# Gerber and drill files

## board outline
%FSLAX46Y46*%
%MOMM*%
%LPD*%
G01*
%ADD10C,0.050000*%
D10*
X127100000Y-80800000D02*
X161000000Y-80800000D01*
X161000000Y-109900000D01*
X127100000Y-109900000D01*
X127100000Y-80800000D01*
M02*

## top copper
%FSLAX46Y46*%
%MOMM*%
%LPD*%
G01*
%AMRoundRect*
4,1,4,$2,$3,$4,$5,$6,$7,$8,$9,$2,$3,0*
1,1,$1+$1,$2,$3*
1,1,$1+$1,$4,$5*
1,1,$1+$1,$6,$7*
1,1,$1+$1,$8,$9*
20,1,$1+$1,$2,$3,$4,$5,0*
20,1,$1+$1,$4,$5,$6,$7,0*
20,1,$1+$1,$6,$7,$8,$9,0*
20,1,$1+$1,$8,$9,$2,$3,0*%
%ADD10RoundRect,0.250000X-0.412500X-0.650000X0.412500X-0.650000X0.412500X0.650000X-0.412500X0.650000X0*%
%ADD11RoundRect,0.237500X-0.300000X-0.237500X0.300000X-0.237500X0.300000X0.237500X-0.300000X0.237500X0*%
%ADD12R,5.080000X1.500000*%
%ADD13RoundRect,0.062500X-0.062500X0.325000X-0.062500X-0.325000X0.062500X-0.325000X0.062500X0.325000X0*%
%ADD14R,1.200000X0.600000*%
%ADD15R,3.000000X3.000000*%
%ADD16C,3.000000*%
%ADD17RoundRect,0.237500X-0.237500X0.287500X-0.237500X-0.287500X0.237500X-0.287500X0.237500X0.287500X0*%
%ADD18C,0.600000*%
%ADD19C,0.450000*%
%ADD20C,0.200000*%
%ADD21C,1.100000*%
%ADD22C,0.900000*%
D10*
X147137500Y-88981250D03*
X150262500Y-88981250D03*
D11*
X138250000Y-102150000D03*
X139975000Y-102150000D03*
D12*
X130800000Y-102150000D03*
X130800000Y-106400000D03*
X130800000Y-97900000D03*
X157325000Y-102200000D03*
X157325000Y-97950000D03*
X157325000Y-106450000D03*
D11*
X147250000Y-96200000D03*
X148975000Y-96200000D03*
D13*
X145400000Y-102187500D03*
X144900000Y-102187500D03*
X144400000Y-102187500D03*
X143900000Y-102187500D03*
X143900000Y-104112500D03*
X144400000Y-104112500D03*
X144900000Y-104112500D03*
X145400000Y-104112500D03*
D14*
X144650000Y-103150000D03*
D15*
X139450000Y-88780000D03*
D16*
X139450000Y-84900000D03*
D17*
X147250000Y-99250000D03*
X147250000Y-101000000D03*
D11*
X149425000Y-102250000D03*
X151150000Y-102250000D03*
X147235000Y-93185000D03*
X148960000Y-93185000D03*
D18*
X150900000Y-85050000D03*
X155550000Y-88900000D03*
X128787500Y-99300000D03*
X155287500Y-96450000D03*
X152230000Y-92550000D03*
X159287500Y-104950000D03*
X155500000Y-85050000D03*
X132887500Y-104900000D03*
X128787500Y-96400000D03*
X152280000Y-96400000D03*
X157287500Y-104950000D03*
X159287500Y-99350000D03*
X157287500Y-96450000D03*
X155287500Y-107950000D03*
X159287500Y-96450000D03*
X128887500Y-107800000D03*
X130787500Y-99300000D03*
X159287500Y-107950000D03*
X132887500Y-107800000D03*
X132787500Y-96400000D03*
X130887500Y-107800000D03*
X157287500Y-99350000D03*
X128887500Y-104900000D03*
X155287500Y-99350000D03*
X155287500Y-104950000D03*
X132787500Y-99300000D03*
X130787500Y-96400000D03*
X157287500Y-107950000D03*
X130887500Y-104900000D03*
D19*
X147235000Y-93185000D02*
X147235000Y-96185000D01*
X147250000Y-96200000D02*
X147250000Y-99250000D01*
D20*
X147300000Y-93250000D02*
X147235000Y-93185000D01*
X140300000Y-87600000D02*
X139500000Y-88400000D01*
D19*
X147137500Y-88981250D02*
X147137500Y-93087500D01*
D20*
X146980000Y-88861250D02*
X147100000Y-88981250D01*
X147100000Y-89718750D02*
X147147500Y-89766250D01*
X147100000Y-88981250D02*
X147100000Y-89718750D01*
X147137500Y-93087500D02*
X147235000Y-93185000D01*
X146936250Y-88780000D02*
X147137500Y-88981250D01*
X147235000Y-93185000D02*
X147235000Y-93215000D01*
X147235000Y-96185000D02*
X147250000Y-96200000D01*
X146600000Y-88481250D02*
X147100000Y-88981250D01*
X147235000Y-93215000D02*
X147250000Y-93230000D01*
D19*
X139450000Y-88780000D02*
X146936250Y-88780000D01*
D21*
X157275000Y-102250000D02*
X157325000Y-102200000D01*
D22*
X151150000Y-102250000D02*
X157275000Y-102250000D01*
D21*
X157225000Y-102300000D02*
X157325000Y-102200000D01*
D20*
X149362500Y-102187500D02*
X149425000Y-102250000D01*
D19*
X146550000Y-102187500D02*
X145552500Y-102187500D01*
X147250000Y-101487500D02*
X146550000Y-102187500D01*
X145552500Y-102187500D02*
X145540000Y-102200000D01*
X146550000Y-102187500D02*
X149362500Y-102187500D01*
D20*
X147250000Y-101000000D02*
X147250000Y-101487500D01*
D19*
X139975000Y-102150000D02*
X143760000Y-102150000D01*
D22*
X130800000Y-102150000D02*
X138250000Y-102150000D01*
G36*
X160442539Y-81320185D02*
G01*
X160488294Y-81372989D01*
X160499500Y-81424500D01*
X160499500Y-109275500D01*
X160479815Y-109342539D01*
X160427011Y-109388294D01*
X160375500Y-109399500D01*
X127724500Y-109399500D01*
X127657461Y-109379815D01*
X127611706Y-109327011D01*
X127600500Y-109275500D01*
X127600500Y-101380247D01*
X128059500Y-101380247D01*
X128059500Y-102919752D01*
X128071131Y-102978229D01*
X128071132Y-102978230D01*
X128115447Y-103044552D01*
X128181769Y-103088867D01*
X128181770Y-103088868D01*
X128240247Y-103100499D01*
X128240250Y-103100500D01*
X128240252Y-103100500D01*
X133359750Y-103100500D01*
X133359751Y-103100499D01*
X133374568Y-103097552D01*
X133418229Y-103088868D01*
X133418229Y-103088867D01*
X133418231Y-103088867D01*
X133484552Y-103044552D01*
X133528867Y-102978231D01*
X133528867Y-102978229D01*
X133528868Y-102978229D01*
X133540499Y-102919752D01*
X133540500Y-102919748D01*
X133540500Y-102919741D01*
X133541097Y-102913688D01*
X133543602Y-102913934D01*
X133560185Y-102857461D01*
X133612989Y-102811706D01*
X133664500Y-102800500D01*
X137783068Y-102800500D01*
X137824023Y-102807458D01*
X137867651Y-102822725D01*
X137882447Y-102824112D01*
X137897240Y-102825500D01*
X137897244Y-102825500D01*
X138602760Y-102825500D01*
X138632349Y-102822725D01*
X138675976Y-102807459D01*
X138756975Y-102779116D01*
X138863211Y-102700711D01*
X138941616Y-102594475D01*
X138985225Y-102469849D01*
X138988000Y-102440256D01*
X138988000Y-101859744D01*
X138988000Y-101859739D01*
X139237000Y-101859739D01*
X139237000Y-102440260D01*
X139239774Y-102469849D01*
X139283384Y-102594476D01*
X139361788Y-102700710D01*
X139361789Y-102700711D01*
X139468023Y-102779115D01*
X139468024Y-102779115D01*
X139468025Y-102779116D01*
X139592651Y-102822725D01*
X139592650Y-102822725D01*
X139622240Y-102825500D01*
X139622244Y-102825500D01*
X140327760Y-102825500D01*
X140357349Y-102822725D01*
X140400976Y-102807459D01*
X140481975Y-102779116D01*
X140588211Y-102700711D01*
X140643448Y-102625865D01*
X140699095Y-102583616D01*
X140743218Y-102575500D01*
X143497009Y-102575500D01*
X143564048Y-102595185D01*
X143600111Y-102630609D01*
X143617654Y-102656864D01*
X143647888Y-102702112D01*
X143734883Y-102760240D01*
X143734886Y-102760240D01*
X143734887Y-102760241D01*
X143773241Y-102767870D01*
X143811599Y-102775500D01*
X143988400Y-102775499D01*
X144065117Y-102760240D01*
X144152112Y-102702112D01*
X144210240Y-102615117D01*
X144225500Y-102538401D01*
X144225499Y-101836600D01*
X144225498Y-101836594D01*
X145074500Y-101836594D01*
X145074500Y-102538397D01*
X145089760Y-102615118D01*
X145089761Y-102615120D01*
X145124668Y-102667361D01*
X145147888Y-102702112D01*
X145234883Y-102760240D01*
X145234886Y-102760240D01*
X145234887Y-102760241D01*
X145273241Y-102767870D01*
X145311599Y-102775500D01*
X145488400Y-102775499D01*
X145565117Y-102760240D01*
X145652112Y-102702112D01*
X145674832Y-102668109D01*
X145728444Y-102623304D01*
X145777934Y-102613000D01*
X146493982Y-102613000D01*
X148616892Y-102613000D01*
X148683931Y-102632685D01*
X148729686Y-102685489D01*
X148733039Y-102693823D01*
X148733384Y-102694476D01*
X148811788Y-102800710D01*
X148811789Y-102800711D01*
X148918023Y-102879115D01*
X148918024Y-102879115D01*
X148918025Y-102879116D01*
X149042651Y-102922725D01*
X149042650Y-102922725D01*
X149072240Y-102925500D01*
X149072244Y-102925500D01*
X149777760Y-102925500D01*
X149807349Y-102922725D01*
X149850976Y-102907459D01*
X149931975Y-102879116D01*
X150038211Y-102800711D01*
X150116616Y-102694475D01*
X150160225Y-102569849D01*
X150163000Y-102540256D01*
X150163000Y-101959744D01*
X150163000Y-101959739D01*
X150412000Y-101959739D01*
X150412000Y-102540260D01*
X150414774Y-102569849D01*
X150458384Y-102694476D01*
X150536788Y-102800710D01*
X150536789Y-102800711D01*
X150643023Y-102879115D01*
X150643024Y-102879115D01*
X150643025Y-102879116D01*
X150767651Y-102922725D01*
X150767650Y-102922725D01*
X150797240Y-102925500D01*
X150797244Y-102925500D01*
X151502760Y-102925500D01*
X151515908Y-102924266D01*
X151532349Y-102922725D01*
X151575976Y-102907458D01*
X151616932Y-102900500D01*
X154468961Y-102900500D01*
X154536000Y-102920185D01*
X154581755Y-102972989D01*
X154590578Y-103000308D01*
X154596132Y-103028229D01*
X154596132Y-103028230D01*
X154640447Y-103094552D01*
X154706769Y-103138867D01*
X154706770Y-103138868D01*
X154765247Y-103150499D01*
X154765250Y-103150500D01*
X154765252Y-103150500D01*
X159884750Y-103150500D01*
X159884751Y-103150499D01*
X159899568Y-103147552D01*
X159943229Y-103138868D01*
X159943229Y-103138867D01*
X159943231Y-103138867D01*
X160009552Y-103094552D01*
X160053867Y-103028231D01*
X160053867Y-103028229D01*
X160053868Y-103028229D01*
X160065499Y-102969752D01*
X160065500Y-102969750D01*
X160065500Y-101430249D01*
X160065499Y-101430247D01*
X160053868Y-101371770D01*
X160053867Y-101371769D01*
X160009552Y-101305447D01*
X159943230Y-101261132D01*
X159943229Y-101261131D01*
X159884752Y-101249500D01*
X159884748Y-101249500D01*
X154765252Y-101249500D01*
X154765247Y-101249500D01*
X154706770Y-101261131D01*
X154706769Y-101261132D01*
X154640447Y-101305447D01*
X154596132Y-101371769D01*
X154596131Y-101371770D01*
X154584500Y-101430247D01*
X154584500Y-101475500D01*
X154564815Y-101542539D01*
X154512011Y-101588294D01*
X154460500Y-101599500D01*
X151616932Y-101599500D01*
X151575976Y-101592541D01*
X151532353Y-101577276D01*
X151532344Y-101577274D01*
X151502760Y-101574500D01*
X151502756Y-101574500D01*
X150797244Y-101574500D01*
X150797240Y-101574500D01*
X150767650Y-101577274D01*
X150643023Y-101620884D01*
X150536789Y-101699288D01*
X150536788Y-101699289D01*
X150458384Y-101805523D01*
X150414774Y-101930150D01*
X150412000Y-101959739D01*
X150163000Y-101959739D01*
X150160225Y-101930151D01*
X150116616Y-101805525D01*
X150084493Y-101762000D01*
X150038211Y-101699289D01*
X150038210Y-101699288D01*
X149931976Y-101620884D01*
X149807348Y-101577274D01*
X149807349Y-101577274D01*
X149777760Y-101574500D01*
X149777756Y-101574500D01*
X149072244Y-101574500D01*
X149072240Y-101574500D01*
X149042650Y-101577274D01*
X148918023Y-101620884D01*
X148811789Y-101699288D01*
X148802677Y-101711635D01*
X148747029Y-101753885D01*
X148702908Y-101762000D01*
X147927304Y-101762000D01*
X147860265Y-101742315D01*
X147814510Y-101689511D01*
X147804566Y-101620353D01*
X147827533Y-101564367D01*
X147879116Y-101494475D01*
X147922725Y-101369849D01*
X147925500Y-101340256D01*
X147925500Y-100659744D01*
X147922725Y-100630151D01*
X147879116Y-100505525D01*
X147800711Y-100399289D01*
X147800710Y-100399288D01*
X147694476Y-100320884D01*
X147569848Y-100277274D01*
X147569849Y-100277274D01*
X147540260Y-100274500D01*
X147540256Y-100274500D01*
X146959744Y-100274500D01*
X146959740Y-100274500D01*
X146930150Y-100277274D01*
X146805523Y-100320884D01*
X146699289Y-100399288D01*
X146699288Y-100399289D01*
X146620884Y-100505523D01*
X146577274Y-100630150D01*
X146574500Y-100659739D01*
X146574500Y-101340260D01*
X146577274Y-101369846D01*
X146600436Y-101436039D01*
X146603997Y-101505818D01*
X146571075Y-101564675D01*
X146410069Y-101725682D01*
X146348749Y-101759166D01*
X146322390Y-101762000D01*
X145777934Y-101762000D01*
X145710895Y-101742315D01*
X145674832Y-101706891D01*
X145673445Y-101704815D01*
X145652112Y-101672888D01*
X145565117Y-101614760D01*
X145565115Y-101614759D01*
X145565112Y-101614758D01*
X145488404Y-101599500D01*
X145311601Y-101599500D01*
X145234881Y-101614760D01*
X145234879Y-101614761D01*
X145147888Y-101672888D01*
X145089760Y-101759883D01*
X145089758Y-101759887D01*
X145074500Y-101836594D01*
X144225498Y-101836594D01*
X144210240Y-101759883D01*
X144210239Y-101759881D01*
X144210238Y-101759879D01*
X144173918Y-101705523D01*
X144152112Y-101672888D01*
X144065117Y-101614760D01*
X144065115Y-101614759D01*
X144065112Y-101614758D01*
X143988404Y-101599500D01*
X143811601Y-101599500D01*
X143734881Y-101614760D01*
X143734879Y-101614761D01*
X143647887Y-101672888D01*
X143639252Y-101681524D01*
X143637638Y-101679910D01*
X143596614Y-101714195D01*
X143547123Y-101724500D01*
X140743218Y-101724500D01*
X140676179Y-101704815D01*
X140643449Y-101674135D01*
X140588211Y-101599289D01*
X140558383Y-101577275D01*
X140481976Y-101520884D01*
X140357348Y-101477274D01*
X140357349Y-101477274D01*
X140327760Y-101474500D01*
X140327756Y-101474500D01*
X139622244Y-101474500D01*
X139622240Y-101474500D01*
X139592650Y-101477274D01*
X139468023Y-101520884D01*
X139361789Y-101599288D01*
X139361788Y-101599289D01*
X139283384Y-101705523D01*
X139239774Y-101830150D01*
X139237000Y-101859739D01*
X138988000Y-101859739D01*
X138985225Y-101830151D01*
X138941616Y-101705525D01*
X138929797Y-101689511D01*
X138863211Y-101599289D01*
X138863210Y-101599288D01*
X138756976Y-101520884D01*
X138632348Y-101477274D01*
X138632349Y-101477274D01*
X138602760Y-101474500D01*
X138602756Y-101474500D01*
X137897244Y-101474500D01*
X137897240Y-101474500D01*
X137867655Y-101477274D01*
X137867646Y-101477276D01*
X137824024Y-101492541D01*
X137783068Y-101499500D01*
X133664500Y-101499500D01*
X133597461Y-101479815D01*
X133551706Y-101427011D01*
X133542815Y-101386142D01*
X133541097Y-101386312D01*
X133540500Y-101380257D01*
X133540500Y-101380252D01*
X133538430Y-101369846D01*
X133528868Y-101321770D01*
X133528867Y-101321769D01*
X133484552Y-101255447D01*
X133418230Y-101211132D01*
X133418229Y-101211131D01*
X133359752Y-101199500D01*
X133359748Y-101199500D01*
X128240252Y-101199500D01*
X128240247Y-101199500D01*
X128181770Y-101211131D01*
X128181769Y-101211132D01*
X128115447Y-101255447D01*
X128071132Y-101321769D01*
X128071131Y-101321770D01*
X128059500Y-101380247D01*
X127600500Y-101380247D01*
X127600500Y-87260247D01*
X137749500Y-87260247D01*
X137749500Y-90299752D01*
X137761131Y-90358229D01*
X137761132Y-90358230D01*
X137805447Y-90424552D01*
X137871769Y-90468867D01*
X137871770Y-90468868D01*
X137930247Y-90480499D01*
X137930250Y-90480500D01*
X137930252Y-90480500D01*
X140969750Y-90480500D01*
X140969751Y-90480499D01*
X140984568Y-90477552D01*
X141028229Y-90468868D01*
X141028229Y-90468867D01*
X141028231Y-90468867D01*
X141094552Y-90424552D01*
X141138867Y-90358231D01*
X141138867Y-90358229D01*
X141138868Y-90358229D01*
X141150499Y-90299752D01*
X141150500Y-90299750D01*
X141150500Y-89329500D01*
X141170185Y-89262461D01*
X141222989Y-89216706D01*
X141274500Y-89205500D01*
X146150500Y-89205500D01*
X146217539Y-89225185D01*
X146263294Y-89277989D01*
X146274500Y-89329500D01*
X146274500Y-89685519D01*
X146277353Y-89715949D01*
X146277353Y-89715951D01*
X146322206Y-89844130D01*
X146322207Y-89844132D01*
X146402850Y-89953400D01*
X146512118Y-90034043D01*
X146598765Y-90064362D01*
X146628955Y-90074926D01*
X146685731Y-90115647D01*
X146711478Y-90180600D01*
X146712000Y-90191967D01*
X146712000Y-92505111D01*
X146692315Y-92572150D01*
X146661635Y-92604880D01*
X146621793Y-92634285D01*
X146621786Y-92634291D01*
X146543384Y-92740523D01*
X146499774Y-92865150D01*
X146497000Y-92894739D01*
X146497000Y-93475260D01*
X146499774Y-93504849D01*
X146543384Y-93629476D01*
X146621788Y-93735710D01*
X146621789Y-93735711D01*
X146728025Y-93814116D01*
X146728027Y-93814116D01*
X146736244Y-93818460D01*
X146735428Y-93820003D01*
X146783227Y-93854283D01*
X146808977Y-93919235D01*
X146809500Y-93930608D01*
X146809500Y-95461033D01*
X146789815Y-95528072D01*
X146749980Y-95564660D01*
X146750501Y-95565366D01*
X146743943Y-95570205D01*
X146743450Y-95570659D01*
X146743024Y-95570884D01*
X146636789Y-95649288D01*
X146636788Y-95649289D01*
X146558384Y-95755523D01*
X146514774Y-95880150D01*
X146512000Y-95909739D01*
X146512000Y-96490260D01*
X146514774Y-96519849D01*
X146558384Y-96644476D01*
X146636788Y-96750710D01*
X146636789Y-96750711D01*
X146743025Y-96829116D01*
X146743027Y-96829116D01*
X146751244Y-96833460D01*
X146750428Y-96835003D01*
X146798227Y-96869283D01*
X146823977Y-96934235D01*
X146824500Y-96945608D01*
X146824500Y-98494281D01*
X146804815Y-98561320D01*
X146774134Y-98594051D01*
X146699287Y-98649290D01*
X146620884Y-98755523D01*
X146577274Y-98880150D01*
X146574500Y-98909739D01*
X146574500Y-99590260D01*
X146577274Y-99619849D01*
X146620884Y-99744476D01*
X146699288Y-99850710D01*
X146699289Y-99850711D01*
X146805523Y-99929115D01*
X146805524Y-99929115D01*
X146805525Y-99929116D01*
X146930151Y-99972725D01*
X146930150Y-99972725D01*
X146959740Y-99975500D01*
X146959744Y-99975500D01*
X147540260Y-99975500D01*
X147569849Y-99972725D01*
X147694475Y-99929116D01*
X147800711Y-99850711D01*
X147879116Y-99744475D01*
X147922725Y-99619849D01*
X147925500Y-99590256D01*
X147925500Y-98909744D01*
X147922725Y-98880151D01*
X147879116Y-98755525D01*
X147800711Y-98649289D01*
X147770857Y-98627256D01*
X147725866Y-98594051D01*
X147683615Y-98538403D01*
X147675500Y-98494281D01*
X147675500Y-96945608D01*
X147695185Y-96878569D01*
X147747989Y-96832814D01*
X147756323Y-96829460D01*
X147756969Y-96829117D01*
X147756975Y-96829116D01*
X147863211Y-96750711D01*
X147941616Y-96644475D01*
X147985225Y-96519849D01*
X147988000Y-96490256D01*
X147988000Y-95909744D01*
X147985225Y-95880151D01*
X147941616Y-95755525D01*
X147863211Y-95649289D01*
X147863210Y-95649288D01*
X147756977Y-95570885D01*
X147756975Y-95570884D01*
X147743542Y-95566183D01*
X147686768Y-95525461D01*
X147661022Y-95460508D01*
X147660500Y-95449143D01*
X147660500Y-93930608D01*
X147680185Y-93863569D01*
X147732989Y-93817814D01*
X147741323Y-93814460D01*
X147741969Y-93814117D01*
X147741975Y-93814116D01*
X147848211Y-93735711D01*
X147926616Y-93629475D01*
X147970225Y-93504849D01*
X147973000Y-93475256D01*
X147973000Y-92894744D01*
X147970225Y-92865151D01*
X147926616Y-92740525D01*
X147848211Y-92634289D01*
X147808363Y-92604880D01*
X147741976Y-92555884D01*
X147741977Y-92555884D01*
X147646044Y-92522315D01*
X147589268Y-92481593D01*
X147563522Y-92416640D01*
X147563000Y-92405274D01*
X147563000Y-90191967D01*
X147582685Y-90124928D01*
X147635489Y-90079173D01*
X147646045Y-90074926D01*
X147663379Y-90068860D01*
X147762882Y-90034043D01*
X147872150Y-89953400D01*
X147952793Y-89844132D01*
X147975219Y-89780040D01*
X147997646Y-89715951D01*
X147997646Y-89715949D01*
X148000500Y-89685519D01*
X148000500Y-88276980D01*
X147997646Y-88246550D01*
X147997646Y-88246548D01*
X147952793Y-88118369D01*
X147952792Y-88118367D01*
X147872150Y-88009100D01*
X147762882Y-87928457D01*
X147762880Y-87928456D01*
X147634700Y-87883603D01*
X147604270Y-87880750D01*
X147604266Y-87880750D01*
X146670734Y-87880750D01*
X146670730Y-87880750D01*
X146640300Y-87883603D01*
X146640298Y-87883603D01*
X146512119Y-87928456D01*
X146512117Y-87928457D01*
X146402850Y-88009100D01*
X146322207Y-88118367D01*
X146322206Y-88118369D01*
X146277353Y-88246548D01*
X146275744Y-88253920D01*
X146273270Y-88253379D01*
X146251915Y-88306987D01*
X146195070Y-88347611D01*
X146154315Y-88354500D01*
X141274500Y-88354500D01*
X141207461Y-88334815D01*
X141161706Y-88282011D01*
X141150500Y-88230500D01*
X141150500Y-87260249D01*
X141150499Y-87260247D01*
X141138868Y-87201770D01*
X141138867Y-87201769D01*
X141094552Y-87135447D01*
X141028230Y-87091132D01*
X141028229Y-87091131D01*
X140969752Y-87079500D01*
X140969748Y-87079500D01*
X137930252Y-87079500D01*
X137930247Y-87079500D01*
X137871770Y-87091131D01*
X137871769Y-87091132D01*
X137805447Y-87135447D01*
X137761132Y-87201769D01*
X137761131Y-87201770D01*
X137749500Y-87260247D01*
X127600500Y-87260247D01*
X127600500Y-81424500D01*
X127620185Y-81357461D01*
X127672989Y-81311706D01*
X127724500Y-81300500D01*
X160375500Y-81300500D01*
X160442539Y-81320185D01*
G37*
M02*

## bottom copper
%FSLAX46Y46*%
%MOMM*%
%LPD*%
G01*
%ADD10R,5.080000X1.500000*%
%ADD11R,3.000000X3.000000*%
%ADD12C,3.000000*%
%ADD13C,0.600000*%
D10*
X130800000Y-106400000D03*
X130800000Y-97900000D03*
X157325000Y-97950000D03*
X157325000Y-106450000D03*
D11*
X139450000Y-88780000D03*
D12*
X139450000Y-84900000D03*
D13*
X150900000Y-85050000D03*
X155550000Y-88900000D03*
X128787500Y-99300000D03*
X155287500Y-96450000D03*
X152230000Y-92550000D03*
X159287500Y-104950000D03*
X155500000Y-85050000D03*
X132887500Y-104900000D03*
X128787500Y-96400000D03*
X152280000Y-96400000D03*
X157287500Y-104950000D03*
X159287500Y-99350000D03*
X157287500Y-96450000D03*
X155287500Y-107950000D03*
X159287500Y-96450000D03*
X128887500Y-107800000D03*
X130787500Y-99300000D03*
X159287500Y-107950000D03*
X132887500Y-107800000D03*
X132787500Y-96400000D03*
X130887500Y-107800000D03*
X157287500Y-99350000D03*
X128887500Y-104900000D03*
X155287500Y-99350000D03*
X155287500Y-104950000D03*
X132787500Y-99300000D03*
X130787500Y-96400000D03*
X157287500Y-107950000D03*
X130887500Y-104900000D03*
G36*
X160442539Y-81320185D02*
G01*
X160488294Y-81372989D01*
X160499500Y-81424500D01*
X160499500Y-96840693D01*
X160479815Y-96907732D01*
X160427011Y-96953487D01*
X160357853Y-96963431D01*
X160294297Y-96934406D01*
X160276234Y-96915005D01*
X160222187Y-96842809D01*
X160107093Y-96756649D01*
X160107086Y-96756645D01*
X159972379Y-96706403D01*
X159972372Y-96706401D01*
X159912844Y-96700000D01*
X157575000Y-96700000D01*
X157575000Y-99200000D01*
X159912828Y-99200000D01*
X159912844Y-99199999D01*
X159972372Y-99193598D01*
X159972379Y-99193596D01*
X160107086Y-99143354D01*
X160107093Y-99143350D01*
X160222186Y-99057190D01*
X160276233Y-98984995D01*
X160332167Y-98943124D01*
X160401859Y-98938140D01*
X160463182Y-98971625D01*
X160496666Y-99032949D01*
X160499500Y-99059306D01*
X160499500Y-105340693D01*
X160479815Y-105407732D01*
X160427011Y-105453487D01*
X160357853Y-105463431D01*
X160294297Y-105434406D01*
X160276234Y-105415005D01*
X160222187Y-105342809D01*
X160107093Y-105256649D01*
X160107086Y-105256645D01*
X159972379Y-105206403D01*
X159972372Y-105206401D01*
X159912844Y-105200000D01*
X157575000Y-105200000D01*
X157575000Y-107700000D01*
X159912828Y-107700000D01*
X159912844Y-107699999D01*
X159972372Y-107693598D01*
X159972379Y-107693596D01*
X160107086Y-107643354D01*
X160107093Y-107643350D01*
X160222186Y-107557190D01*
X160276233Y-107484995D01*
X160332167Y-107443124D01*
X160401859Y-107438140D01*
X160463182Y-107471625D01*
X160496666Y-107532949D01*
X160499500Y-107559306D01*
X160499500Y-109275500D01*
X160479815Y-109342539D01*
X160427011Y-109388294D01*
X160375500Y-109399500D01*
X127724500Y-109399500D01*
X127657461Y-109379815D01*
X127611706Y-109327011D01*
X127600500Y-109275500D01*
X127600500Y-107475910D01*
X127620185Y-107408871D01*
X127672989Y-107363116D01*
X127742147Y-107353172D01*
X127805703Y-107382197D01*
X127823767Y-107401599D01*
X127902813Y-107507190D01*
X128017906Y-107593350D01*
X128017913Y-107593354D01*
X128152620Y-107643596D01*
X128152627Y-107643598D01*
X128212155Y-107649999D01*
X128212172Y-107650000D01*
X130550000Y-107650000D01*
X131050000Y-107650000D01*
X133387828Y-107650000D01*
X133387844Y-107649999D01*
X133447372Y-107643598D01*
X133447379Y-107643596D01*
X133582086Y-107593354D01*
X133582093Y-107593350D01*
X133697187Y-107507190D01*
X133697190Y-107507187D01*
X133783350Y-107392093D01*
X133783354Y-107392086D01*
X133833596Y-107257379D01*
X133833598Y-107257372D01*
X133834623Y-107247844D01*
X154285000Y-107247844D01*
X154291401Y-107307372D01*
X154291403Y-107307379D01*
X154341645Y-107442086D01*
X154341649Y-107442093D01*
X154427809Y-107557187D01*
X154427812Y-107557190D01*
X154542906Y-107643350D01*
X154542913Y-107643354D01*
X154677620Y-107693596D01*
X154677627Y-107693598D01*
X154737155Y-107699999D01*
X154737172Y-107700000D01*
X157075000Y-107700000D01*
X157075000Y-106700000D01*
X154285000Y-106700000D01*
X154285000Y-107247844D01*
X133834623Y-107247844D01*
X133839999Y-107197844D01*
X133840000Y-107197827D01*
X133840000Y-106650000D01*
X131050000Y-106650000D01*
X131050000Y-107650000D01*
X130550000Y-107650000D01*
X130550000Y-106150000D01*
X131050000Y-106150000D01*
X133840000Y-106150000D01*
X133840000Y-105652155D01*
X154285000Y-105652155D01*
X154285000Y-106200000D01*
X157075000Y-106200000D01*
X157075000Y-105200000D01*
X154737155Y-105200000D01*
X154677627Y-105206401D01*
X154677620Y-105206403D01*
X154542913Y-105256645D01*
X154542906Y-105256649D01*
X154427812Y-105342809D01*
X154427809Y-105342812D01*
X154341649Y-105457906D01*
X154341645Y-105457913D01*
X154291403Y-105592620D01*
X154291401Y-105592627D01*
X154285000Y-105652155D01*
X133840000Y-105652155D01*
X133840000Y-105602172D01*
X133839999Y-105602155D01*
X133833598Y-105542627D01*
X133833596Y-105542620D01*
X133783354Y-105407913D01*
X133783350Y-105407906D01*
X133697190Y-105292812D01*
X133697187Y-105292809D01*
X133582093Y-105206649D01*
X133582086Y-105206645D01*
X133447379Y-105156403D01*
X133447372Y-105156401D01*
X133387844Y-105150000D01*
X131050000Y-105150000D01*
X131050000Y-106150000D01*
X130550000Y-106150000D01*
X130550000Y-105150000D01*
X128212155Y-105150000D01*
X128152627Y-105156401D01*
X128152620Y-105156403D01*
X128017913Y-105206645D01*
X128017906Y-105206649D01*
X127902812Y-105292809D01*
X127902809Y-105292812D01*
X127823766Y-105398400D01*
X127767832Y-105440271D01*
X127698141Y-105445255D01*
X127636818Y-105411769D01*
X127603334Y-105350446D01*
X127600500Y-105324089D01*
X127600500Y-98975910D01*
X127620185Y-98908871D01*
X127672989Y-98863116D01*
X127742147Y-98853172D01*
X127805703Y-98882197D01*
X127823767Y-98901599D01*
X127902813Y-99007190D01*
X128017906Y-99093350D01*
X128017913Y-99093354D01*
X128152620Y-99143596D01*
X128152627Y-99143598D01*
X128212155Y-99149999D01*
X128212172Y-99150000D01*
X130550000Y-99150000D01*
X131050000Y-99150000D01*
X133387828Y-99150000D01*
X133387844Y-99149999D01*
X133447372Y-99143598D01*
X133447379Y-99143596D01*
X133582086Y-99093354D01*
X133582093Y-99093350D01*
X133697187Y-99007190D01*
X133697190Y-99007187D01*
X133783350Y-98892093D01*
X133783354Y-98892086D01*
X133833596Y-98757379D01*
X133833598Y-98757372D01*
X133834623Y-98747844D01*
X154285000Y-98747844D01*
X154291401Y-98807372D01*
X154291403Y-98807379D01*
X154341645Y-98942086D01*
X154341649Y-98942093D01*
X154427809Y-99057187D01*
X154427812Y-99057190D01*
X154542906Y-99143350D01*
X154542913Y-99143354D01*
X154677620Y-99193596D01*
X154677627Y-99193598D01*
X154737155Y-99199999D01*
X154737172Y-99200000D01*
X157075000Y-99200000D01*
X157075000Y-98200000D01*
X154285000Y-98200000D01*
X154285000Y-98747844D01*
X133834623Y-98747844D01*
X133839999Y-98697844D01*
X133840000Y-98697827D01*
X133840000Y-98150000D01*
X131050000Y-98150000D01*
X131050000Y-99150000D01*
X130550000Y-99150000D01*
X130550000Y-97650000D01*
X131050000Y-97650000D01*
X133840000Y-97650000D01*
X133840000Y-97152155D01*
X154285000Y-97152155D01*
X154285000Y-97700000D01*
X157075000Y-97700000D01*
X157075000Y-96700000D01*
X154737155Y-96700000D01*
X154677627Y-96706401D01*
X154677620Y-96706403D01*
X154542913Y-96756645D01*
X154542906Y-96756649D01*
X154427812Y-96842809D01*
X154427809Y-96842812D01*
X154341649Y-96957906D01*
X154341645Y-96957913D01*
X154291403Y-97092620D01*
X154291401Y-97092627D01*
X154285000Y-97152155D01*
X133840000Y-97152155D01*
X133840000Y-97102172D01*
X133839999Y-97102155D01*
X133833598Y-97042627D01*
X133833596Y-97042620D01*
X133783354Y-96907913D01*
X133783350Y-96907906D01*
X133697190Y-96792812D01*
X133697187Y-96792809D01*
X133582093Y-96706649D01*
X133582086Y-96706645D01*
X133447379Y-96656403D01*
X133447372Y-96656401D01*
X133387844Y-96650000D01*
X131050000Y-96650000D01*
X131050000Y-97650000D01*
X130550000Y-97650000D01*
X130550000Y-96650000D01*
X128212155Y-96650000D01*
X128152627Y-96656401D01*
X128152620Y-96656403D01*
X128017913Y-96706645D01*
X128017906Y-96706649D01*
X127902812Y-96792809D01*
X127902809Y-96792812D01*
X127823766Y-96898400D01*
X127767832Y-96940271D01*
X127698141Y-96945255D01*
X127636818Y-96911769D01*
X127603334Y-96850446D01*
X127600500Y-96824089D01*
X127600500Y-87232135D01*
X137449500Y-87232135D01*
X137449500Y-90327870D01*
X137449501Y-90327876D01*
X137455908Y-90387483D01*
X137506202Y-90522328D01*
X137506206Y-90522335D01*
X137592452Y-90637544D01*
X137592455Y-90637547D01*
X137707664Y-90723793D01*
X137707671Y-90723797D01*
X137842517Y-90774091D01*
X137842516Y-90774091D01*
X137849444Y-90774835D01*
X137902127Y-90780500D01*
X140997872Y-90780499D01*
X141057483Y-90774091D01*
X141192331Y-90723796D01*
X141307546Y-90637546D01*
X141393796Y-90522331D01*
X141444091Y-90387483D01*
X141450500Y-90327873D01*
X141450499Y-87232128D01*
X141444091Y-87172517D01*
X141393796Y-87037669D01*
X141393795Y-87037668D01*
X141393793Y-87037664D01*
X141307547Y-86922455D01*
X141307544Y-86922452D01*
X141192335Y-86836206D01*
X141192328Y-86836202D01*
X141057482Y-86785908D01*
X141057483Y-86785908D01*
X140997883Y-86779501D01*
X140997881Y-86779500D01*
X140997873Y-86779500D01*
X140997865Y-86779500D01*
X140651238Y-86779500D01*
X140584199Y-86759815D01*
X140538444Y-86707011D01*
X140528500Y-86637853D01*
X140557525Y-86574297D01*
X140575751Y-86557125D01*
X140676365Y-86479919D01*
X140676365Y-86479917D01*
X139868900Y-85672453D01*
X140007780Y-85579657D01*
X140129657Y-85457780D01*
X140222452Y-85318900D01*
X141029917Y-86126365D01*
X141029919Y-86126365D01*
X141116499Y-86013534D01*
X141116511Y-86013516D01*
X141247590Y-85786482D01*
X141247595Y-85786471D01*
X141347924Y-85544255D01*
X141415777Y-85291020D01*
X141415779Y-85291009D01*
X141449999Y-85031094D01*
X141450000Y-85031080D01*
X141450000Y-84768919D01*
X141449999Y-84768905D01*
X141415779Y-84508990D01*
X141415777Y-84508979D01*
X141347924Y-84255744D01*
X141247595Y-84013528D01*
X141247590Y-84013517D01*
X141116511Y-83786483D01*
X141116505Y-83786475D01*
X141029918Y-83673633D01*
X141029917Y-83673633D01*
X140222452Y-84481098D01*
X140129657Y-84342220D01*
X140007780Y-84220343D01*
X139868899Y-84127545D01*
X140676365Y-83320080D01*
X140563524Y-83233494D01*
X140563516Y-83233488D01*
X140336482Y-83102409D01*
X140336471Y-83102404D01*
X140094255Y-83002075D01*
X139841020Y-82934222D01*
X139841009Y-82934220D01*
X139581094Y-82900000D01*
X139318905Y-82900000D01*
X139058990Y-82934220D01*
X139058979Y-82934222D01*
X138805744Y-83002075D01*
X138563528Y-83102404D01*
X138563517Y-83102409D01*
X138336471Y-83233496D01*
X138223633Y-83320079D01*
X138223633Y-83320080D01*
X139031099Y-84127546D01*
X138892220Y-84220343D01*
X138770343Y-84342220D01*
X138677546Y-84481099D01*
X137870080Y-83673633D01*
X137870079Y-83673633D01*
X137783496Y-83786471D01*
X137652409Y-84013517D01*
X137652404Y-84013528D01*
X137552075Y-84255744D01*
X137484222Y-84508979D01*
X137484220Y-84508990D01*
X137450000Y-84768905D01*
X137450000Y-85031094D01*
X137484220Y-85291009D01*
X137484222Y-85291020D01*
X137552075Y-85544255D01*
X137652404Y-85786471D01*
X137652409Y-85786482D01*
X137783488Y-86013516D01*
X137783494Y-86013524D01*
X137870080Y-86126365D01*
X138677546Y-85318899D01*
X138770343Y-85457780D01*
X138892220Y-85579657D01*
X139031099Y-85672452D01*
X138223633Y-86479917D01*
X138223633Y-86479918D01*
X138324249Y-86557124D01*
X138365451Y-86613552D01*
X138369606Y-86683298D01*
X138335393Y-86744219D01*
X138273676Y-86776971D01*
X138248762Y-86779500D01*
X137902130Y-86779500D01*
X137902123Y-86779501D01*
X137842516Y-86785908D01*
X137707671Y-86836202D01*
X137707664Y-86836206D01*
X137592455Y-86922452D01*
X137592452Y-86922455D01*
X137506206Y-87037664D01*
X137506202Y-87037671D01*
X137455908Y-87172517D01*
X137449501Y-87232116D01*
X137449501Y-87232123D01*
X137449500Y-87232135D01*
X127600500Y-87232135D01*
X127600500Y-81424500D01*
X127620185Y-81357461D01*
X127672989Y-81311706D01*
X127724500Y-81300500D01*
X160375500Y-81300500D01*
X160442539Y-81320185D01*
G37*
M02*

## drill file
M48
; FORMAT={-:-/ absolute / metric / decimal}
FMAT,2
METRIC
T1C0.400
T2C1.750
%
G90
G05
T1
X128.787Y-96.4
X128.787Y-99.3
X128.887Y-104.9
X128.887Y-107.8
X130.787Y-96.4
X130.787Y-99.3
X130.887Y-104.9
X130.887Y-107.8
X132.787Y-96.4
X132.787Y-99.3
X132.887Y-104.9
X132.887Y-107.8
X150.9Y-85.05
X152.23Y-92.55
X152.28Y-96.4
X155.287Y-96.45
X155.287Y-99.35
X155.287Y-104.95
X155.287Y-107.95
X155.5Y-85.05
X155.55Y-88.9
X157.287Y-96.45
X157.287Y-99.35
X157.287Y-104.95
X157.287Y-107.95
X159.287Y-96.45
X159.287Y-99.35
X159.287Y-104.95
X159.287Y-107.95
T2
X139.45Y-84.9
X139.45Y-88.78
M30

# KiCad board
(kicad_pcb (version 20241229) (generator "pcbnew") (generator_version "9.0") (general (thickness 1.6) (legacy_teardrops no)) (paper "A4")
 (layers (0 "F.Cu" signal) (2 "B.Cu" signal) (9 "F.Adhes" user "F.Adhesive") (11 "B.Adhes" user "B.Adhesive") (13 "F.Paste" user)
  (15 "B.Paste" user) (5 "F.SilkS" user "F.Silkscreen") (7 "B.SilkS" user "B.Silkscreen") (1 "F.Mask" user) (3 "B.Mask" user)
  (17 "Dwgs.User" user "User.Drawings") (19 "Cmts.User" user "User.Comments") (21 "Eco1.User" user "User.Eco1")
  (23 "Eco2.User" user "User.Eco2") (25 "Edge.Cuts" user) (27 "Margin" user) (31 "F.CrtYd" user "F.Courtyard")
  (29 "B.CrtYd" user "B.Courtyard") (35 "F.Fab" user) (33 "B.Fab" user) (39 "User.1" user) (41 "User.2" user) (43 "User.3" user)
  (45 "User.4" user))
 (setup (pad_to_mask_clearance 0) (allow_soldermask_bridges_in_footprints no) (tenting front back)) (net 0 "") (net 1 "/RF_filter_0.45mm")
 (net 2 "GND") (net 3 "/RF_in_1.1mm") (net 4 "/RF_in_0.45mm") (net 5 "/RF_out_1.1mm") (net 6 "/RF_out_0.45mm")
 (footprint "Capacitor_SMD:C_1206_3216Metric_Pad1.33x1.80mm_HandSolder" (layer "F.Cu") (at 148.7 88.98125)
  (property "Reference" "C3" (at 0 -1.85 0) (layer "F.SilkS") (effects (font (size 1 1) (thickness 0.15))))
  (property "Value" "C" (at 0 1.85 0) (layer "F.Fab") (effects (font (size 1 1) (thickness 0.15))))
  (pad "1" smd roundrect (at -1.5625 0) (size 1.325 1.8) (layers "F.Cu" "F.Mask" "F.Paste") (roundrect_rratio 0.188679)
   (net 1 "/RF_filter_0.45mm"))
  (pad "2" smd roundrect (at 1.5625 0) (size 1.325 1.8) (layers "F.Cu" "F.Mask" "F.Paste") (roundrect_rratio 0.188679) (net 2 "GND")))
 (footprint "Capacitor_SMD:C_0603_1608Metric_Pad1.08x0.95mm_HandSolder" (layer "F.Cu") (at 139.1125 102.15)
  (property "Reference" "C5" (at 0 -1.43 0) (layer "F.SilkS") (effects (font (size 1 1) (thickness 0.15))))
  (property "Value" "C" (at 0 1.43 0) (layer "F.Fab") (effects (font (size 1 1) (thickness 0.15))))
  (pad "1" smd roundrect (at -0.8625 0) (size 1.075 0.95) (layers "F.Cu" "F.Mask" "F.Paste") (roundrect_rratio 0.25) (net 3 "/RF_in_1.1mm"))
  (pad "2" smd roundrect (at 0.8625 0) (size 1.075 0.95) (layers "F.Cu" "F.Mask" "F.Paste") (roundrect_rratio 0.25) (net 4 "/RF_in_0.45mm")))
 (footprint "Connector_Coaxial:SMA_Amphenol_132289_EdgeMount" (layer "F.Cu") (at 130.8 102.15 180)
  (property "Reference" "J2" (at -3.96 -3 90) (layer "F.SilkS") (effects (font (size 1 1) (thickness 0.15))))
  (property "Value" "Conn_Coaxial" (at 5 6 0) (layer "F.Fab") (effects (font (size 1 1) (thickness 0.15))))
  (pad "1" smd rect (at 0 0 270) (size 1.5 5.08) (layers "F.Cu" "F.Mask" "F.Paste") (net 3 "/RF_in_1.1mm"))
  (pad "2" smd rect (at 0 -4.25 270) (size 1.5 5.08) (layers "F.Cu" "F.Mask" "F.Paste") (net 2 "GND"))
  (pad "2" smd rect (at 0 -4.25 270) (size 1.5 5.08) (layers "B.Cu" "B.Mask" "B.Paste") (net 2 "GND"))
  (pad "2" smd rect (at 0 4.25 270) (size 1.5 5.08) (layers "F.Cu" "F.Mask" "F.Paste") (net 2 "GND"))
  (pad "2" smd rect (at 0 4.25 270) (size 1.5 5.08) (layers "B.Cu" "B.Mask" "B.Paste") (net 2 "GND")))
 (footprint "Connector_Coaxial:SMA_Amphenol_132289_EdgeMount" (layer "F.Cu") (at 157.325 102.2)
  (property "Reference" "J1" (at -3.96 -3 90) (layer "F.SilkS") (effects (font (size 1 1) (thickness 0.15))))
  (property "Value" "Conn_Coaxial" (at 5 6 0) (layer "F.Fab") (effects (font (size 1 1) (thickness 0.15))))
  (pad "1" smd rect (at 0 0 90) (size 1.5 5.08) (layers "F.Cu" "F.Mask" "F.Paste") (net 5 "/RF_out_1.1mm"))
  (pad "2" smd rect (at 0 -4.25 90) (size 1.5 5.08) (layers "F.Cu" "F.Mask" "F.Paste") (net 2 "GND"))
  (pad "2" smd rect (at 0 -4.25 90) (size 1.5 5.08) (layers "B.Cu" "B.Mask" "B.Paste") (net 2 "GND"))
  (pad "2" smd rect (at 0 4.25 90) (size 1.5 5.08) (layers "F.Cu" "F.Mask" "F.Paste") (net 2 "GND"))
  (pad "2" smd rect (at 0 4.25 90) (size 1.5 5.08) (layers "B.Cu" "B.Mask" "B.Paste") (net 2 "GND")))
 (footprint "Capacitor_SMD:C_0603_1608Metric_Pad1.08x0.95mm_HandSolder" (layer "F.Cu") (at 148.1125 96.2)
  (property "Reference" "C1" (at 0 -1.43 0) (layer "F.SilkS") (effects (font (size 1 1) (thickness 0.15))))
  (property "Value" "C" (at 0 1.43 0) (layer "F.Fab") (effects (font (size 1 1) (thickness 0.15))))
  (pad "1" smd roundrect (at -0.8625 0) (size 1.075 0.95) (layers "F.Cu" "F.Mask" "F.Paste") (roundrect_rratio 0.25)
   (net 1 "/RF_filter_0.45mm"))
  (pad "2" smd roundrect (at 0.8625 0) (size 1.075 0.95) (layers "F.Cu" "F.Mask" "F.Paste") (roundrect_rratio 0.25) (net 2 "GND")))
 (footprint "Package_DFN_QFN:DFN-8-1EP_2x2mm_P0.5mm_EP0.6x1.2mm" (layer "F.Cu") (at 144.65 103.15 -90)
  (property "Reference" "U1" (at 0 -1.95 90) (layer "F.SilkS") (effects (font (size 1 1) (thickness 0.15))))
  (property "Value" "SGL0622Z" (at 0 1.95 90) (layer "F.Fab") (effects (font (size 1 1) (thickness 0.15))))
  (pad "" smd roundrect (at -0.15 -0.3 270) (size 0.24 0.48) (layers "F.Paste") (roundrect_rratio 0.25))
  (pad "" smd roundrect (at -0.15 0.3 270) (size 0.24 0.48) (layers "F.Paste") (roundrect_rratio 0.25))
  (pad "" smd roundrect (at 0.15 -0.3 270) (size 0.24 0.48) (layers "F.Paste") (roundrect_rratio 0.25))
  (pad "" smd roundrect (at 0.15 0.3 270) (size 0.24 0.48) (layers "F.Paste") (roundrect_rratio 0.25))
  (pad "1" smd roundrect (at -0.9625 -0.75 270) (size 0.775 0.25) (layers "F.Cu" "F.Mask" "F.Paste") (roundrect_rratio 0.25)
   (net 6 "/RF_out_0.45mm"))
  (pad "2" smd roundrect (at -0.9625 -0.25 270) (size 0.775 0.25) (layers "F.Cu" "F.Mask" "F.Paste") (roundrect_rratio 0.25) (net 2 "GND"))
  (pad "3" smd roundrect (at -0.9625 0.25 270) (size 0.775 0.25) (layers "F.Cu" "F.Mask" "F.Paste") (roundrect_rratio 0.25) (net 2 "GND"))
  (pad "4" smd roundrect (at -0.9625 0.75 270) (size 0.775 0.25) (layers "F.Cu" "F.Mask" "F.Paste") (roundrect_rratio 0.25)
   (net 4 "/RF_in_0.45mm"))
  (pad "5" smd roundrect (at 0.9625 0.75 270) (size 0.775 0.25) (layers "F.Cu" "F.Mask" "F.Paste") (roundrect_rratio 0.25) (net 2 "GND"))
  (pad "6" smd roundrect (at 0.9625 0.25 270) (size 0.775 0.25) (layers "F.Cu" "F.Mask" "F.Paste") (roundrect_rratio 0.25) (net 2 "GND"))
  (pad "7" smd roundrect (at 0.9625 -0.25 270) (size 0.775 0.25) (layers "F.Cu" "F.Mask" "F.Paste") (roundrect_rratio 0.25) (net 2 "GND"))
  (pad "8" smd roundrect (at 0.9625 -0.75 270) (size 0.775 0.25) (layers "F.Cu" "F.Mask" "F.Paste") (roundrect_rratio 0.25) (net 2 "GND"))
  (pad "9" smd rect (at 0 0 270) (size 0.6 1.2) (layers "F.Cu" "F.Mask") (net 2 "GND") (zone_connect 2)))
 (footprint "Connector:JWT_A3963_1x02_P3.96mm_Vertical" (layer "F.Cu") (at 139.45 88.78 90)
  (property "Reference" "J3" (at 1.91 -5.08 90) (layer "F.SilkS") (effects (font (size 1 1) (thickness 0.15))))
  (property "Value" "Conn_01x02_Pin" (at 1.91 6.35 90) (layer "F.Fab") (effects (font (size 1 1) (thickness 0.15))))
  (pad "1" thru_hole rect (at 0 0 90) (size 3 3) (drill 1.75) (layers "*.Cu" "*.Mask") (remove_unused_layers no) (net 1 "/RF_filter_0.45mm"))
  (pad "2" thru_hole circle (at 3.88 0 90) (size 3 3) (drill 1.75) (layers "*.Cu" "*.Mask") (remove_unused_layers no) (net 2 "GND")))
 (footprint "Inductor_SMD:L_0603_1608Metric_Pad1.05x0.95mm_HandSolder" (layer "F.Cu") (at 147.25 100.125 -90)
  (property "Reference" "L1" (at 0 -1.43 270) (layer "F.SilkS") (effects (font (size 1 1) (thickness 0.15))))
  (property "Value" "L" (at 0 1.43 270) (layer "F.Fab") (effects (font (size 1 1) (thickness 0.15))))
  (pad "1" smd roundrect (at -0.875 0 270) (size 1.05 0.95) (layers "F.Cu" "F.Mask" "F.Paste") (roundrect_rratio 0.25)
   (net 1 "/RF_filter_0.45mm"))
  (pad "2" smd roundrect (at 0.875 0 270) (size 1.05 0.95) (layers "F.Cu" "F.Mask" "F.Paste") (roundrect_rratio 0.25)
   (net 6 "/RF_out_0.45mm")))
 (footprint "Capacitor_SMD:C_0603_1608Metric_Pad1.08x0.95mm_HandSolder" (layer "F.Cu") (at 150.2875 102.25)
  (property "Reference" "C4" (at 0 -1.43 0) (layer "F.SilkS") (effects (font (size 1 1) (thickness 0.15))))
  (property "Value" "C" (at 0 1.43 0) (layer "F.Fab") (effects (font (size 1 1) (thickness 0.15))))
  (pad "1" smd roundrect (at -0.8625 0) (size 1.075 0.95) (layers "F.Cu" "F.Mask" "F.Paste") (roundrect_rratio 0.25)
   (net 6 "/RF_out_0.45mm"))
  (pad "2" smd roundrect (at 0.8625 0) (size 1.075 0.95) (layers "F.Cu" "F.Mask" "F.Paste") (roundrect_rratio 0.25) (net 5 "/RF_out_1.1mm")))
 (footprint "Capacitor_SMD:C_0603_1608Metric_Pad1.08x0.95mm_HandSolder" (layer "F.Cu") (at 148.0975 93.185)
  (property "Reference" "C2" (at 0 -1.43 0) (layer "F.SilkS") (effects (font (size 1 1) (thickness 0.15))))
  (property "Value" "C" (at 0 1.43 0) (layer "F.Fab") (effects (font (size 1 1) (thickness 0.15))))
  (pad "1" smd roundrect (at -0.8625 0) (size 1.075 0.95) (layers "F.Cu" "F.Mask" "F.Paste") (roundrect_rratio 0.25)
   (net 1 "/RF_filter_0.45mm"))
  (pad "2" smd roundrect (at 0.8625 0) (size 1.075 0.95) (layers "F.Cu" "F.Mask" "F.Paste") (roundrect_rratio 0.25) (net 2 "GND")))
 (gr_rect (start 127.1 80.8) (end 161 109.9) (stroke (width 0.05) (type solid)) (fill no) (layer "Edge.Cuts"))
 (segment (start 147.235 93.185) (end 147.235 96.185) (width 0.45) (layer "F.Cu") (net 1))
 (segment (start 147.25 96.2) (end 147.25 99.25) (width 0.45) (layer "F.Cu") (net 1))
 (segment (start 147.3 93.25) (end 147.235 93.185) (width 0.2) (layer "F.Cu") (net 1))
 (segment (start 140.3 87.6) (end 139.5 88.4) (width 0.2) (layer "F.Cu") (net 1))
 (segment (start 147.1375 88.98125) (end 147.1375 93.0875) (width 0.45) (layer "F.Cu") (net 1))
 (segment (start 146.98 88.86125) (end 147.1 88.98125) (width 0.2) (layer "F.Cu") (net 1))
 (segment (start 147.1 89.71875) (end 147.1475 89.76625) (width 0.2) (layer "F.Cu") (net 1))
 (segment (start 147.1 88.98125) (end 147.1 89.71875) (width 0.2) (layer "F.Cu") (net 1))
 (segment (start 147.1375 93.0875) (end 147.235 93.185) (width 0.2) (layer "F.Cu") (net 1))
 (segment (start 146.93625 88.78) (end 147.1375 88.98125) (width 0.2) (layer "F.Cu") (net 1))
 (segment (start 147.235 93.185) (end 147.235 93.215) (width 0.2) (layer "F.Cu") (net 1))
 (segment (start 147.235 96.185) (end 147.25 96.2) (width 0.2) (layer "F.Cu") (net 1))
 (segment (start 146.6 88.48125) (end 147.1 88.98125) (width 0.2) (layer "F.Cu") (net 1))
 (segment (start 147.235 93.215) (end 147.25 93.23) (width 0.2) (layer "F.Cu") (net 1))
 (segment (start 139.45 88.78) (end 146.93625 88.78) (width 0.45) (layer "F.Cu") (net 1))
 (via (at 150.9 85.05) (size 0.6) (drill 0.4) (layers "F.Cu" "B.Cu") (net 2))
 (via (at 155.55 88.9) (size 0.6) (drill 0.4) (layers "F.Cu" "B.Cu") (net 2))
 (via (at 128.7875 99.3) (size 0.6) (drill 0.4) (layers "F.Cu" "B.Cu") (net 2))
 (via (at 155.2875 96.45) (size 0.6) (drill 0.4) (layers "F.Cu" "B.Cu") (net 2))
 (via (at 152.23 92.55) (size 0.6) (drill 0.4) (layers "F.Cu" "B.Cu") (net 2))
 (via (at 159.2875 104.95) (size 0.6) (drill 0.4) (layers "F.Cu" "B.Cu") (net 2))
 (via (at 155.5 85.05) (size 0.6) (drill 0.4) (layers "F.Cu" "B.Cu") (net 2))
 (via (at 132.8875 104.9) (size 0.6) (drill 0.4) (layers "F.Cu" "B.Cu") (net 2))
 (via (at 128.7875 96.4) (size 0.6) (drill 0.4) (layers "F.Cu" "B.Cu") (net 2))
 (via (at 152.28 96.4) (size 0.6) (drill 0.4) (layers "F.Cu" "B.Cu") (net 2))
 (via (at 157.2875 104.95) (size 0.6) (drill 0.4) (layers "F.Cu" "B.Cu") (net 2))
 (via (at 159.2875 99.35) (size 0.6) (drill 0.4) (layers "F.Cu" "B.Cu") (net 2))
 (via (at 157.2875 96.45) (size 0.6) (drill 0.4) (layers "F.Cu" "B.Cu") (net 2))
 (via (at 155.2875 107.95) (size 0.6) (drill 0.4) (layers "F.Cu" "B.Cu") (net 2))
 (via (at 159.2875 96.45) (size 0.6) (drill 0.4) (layers "F.Cu" "B.Cu") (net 2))
 (via (at 128.8875 107.8) (size 0.6) (drill 0.4) (layers "F.Cu" "B.Cu") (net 2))
 (via (at 130.7875 99.3) (size 0.6) (drill 0.4) (layers "F.Cu" "B.Cu") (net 2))
 (via (at 159.2875 107.95) (size 0.6) (drill 0.4) (layers "F.Cu" "B.Cu") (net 2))
 (via (at 132.8875 107.8) (size 0.6) (drill 0.4) (layers "F.Cu" "B.Cu") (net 2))
 (via (at 132.7875 96.4) (size 0.6) (drill 0.4) (layers "F.Cu" "B.Cu") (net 2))
 (via (at 130.8875 107.8) (size 0.6) (drill 0.4) (layers "F.Cu" "B.Cu") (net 2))
 (via (at 157.2875 99.35) (size 0.6) (drill 0.4) (layers "F.Cu" "B.Cu") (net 2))
 (via (at 128.8875 104.9) (size 0.6) (drill 0.4) (layers "F.Cu" "B.Cu") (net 2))
 (via (at 155.2875 99.35) (size 0.6) (drill 0.4) (layers "F.Cu" "B.Cu") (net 2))
 (via (at 155.2875 104.95) (size 0.6) (drill 0.4) (layers "F.Cu" "B.Cu") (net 2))
 (via (at 132.7875 99.3) (size 0.6) (drill 0.4) (layers "F.Cu" "B.Cu") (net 2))
 (via (at 130.7875 96.4) (size 0.6) (drill 0.4) (layers "F.Cu" "B.Cu") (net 2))
 (via (at 157.2875 107.95) (size 0.6) (drill 0.4) (layers "F.Cu" "B.Cu") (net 2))
 (via (at 130.8875 104.9) (size 0.6) (drill 0.4) (layers "F.Cu" "B.Cu") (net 2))
 (segment (start 157.275 102.25) (end 157.325 102.2) (width 1.1) (layer "F.Cu") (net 5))
 (segment (start 151.15 102.25) (end 157.275 102.25) (width 0.9) (layer "F.Cu") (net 5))
 (segment (start 157.225 102.3) (end 157.325 102.2) (width 1.1) (layer "F.Cu") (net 5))
 (segment (start 149.3625 102.1875) (end 149.425 102.25) (width 0.2) (layer "F.Cu") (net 6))
 (segment (start 146.55 102.1875) (end 145.5525 102.1875) (width 0.45) (layer "F.Cu") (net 6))
 (segment (start 147.25 101.4875) (end 146.55 102.1875) (width 0.45) (layer "F.Cu") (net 6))
 (segment (start 145.5525 102.1875) (end 145.54 102.2) (width 0.45) (layer "F.Cu") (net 6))
 (segment (start 146.55 102.1875) (end 149.3625 102.1875) (width 0.45) (layer "F.Cu") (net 6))
 (segment (start 147.25 101) (end 147.25 101.4875) (width 0.2) (layer "F.Cu") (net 6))
 (segment (start 139.975 102.15) (end 143.76 102.15) (width 0.45) (layer "F.Cu") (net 4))
 (segment (start 130.8 102.15) (end 138.25 102.15) (width 0.9) (layer "F.Cu") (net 3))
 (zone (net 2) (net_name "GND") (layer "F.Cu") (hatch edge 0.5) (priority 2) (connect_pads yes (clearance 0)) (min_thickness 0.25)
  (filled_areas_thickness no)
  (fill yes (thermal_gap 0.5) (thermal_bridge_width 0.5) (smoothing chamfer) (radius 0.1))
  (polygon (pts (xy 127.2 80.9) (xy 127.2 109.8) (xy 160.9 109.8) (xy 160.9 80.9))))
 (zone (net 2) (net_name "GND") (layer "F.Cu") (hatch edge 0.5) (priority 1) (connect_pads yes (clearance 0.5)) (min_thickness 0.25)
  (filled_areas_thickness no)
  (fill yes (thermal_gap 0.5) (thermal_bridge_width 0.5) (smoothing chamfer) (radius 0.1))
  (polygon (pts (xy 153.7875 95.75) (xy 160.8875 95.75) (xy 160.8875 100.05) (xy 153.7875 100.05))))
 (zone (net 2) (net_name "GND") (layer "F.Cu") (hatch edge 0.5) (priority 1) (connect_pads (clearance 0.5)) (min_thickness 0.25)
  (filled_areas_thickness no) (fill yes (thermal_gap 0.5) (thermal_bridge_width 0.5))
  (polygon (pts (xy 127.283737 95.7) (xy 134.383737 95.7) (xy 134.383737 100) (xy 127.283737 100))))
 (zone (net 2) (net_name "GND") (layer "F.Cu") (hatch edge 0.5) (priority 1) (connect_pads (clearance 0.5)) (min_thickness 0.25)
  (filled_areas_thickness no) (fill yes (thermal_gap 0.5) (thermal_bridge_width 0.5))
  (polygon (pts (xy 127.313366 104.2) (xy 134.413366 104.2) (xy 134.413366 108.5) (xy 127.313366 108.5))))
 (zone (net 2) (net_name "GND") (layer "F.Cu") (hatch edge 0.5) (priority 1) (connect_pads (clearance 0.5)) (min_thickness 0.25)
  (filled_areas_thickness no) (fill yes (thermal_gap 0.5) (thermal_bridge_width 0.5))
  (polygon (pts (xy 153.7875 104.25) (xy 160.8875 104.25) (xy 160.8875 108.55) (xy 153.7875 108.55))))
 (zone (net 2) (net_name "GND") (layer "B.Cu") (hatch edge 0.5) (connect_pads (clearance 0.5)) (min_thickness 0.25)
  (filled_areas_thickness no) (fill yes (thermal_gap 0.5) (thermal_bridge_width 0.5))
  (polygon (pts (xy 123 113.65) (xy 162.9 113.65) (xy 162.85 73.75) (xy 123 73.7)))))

